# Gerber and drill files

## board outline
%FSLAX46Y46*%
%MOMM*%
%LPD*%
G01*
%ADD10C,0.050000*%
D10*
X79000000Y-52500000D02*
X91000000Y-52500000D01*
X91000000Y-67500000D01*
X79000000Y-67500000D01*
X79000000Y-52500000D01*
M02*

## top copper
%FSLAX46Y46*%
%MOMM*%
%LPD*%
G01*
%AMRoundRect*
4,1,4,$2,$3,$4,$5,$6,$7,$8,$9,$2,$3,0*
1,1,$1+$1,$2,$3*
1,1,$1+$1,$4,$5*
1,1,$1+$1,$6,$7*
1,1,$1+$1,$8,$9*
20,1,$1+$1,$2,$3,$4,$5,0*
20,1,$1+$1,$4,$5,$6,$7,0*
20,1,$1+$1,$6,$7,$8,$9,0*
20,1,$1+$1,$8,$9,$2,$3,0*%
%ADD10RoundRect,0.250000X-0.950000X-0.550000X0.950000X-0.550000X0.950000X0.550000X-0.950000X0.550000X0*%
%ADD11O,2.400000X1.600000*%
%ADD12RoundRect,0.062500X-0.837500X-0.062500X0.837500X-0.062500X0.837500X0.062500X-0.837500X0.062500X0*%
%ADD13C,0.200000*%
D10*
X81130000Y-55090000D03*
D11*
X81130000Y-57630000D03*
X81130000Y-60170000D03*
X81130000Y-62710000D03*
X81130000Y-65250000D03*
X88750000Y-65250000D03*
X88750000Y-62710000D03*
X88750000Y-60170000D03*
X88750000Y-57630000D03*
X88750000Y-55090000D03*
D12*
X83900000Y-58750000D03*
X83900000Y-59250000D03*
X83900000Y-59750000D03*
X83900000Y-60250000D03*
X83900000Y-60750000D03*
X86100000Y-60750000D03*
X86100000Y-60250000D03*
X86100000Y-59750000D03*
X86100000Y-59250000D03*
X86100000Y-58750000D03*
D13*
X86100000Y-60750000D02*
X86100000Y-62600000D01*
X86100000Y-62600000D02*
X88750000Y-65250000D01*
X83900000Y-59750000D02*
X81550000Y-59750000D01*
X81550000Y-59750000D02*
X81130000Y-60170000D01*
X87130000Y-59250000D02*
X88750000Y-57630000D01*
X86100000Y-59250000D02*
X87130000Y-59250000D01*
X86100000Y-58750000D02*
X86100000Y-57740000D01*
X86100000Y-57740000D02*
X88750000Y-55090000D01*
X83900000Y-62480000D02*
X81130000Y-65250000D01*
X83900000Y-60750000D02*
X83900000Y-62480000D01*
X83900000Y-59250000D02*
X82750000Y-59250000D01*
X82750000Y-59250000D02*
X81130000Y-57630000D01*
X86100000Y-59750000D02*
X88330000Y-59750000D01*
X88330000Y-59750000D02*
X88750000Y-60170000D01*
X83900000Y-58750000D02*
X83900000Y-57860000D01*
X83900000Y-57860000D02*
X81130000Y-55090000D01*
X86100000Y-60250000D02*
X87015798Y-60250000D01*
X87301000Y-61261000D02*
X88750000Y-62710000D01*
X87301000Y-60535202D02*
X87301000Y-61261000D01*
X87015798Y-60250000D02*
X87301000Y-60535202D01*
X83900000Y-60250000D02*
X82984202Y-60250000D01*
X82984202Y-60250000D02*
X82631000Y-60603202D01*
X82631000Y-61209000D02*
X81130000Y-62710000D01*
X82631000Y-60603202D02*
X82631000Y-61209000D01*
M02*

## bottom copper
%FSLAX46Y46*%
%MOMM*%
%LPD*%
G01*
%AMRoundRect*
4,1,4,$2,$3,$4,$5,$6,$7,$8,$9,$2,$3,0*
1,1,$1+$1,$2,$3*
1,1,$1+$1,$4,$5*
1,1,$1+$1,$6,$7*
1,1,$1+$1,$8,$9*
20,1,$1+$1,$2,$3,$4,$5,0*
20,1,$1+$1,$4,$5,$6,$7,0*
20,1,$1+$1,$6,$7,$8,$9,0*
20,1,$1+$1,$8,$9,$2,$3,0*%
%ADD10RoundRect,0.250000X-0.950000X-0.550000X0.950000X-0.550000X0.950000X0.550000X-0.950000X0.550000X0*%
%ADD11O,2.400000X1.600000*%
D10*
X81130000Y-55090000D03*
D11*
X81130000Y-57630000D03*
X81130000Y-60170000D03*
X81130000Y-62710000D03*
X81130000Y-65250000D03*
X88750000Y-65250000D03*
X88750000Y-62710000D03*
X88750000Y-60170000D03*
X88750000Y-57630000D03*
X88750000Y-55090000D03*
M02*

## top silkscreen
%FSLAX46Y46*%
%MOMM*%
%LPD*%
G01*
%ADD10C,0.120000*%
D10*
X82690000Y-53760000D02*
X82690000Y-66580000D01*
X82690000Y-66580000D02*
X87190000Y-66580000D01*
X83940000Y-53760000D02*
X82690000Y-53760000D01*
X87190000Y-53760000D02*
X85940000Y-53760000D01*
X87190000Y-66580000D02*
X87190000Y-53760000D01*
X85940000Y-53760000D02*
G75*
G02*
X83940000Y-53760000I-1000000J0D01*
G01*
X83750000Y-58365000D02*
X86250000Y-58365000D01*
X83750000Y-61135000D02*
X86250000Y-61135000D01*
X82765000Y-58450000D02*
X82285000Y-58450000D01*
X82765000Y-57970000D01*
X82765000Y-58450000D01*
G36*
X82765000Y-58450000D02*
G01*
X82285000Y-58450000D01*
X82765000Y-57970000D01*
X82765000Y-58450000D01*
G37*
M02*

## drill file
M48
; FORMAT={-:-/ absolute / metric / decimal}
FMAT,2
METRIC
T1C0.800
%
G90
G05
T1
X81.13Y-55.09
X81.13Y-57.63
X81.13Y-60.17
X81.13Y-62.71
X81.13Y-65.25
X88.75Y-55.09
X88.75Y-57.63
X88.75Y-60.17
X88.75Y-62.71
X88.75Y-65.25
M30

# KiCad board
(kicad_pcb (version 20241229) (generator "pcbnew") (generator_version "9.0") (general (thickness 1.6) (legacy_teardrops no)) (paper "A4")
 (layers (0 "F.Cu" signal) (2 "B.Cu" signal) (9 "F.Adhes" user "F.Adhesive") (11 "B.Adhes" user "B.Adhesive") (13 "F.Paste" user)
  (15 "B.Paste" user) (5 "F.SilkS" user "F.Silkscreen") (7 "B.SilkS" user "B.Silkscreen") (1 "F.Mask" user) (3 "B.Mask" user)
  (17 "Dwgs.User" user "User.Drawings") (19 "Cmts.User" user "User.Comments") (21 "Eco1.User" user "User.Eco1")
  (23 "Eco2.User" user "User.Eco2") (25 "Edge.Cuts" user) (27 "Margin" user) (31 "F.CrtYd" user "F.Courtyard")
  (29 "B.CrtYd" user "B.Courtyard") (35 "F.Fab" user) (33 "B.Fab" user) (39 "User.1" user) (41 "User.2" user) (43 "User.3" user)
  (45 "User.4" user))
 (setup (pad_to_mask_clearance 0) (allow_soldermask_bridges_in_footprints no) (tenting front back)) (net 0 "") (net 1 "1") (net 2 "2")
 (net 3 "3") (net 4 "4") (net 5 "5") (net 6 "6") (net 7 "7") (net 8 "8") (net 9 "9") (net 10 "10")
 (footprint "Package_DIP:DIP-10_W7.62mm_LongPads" (layer "F.Cu") (at 81.13 55.09)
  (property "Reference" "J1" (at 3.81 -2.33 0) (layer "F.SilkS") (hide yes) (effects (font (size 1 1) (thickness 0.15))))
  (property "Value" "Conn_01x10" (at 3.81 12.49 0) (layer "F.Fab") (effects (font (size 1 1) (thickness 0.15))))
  (fp_line (start 1.56 -1.33) (end 1.56 11.49) (stroke (width 0.12) (type solid)) (layer "F.SilkS"))
  (fp_line (start 1.56 11.49) (end 6.06 11.49) (stroke (width 0.12) (type solid)) (layer "F.SilkS"))
  (fp_line (start 2.81 -1.33) (end 1.56 -1.33) (stroke (width 0.12) (type solid)) (layer "F.SilkS"))
  (fp_line (start 6.06 -1.33) (end 4.81 -1.33) (stroke (width 0.12) (type solid)) (layer "F.SilkS"))
  (fp_line (start 6.06 11.49) (end 6.06 -1.33) (stroke (width 0.12) (type solid)) (layer "F.SilkS"))
  (fp_arc (start 4.81 -1.33) (mid 3.81 -0.33) (end 2.81 -1.33) (stroke (width 0.12) (type solid)) (layer "F.SilkS"))
  (pad "1" thru_hole roundrect (at 0 0) (size 2.4 1.6) (drill 0.8) (layers "*.Cu" "*.Mask") (remove_unused_layers no)
   (roundrect_rratio 0.15625) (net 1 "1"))
  (pad "2" thru_hole oval (at 0 2.54) (size 2.4 1.6) (drill 0.8) (layers "*.Cu" "*.Mask") (remove_unused_layers no) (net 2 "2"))
  (pad "3" thru_hole oval (at 0 5.08) (size 2.4 1.6) (drill 0.8) (layers "*.Cu" "*.Mask") (remove_unused_layers no) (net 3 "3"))
  (pad "4" thru_hole oval (at 0 7.62) (size 2.4 1.6) (drill 0.8) (layers "*.Cu" "*.Mask") (remove_unused_layers no) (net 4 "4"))
  (pad "5" thru_hole oval (at 0 10.16) (size 2.4 1.6) (drill 0.8) (layers "*.Cu" "*.Mask") (remove_unused_layers no) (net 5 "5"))
  (pad "6" thru_hole oval (at 7.62 10.16) (size 2.4 1.6) (drill 0.8) (layers "*.Cu" "*.Mask") (remove_unused_layers no) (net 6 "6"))
  (pad "7" thru_hole oval (at 7.62 7.62) (size 2.4 1.6) (drill 0.8) (layers "*.Cu" "*.Mask") (remove_unused_layers no) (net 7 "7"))
  (pad "8" thru_hole oval (at 7.62 5.08) (size 2.4 1.6) (drill 0.8) (layers "*.Cu" "*.Mask") (remove_unused_layers no) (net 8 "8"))
  (pad "9" thru_hole oval (at 7.62 2.54) (size 2.4 1.6) (drill 0.8) (layers "*.Cu" "*.Mask") (remove_unused_layers no) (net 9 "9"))
  (pad "10" thru_hole oval (at 7.62 0) (size 2.4 1.6) (drill 0.8) (layers "*.Cu" "*.Mask") (remove_unused_layers no) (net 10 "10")))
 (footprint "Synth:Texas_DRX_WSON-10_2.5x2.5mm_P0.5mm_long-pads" (layer "F.Cu") (at 85 59.75)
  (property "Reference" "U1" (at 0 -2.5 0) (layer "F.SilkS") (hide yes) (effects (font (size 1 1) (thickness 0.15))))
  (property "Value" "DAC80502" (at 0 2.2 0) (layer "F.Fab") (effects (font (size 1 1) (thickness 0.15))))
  (fp_line (start -1.25 -1.385) (end 1.25 -1.385) (stroke (width 0.12) (type solid)) (layer "F.SilkS"))
  (fp_line (start -1.25 1.385) (end 1.25 1.385) (stroke (width 0.12) (type solid)) (layer "F.SilkS"))
  (fp_poly
   (pts (xy -2.235 -1.3) (xy -2.715 -1.3) (xy -2.235 -1.78) (xy -2.235 -1.3)) (stroke (width 0.12) (type solid)) (fill yes)
   (layer "F.SilkS"))
  (pad "1" smd roundrect (at -1.1 -1) (size 1.8 0.25) (layers "F.Cu" "F.Mask" "F.Paste") (roundrect_rratio 0.25) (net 1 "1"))
  (pad "2" smd roundrect (at -1.1 -0.5) (size 1.8 0.25) (layers "F.Cu" "F.Mask" "F.Paste") (roundrect_rratio 0.25) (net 2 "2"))
  (pad "3" smd roundrect (at -1.1 0) (size 1.8 0.25) (layers "F.Cu" "F.Mask" "F.Paste") (roundrect_rratio 0.25) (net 3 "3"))
  (pad "4" smd roundrect (at -1.1 0.5) (size 1.8 0.25) (layers "F.Cu" "F.Mask" "F.Paste") (roundrect_rratio 0.25) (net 4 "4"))
  (pad "5" smd roundrect (at -1.1 1) (size 1.8 0.25) (layers "F.Cu" "F.Mask" "F.Paste") (roundrect_rratio 0.25) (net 5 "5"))
  (pad "6" smd roundrect (at 1.1 1) (size 1.8 0.25) (layers "F.Cu" "F.Mask" "F.Paste") (roundrect_rratio 0.25) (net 6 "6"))
  (pad "7" smd roundrect (at 1.1 0.5) (size 1.8 0.25) (layers "F.Cu" "F.Mask" "F.Paste") (roundrect_rratio 0.25) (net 7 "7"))
  (pad "8" smd roundrect (at 1.1 0) (size 1.8 0.25) (layers "F.Cu" "F.Mask" "F.Paste") (roundrect_rratio 0.25) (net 8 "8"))
  (pad "9" smd roundrect (at 1.1 -0.5) (size 1.8 0.25) (layers "F.Cu" "F.Mask" "F.Paste") (roundrect_rratio 0.25) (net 9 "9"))
  (pad "10" smd roundrect (at 1.1 -1) (size 1.8 0.25) (layers "F.Cu" "F.Mask" "F.Paste") (roundrect_rratio 0.25) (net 10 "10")))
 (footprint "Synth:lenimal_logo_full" (layer "B.Cu") (at 85 60 -90)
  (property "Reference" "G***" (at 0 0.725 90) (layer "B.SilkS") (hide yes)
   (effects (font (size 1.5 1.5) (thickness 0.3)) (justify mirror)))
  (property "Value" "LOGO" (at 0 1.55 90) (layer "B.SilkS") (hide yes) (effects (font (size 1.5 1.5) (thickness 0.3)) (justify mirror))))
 (gr_rect (start 79 52.5) (end 91 67.5) (stroke (width 0.05) (type default)) (fill no) (layer "Edge.Cuts"))
 (segment (start 86.1 60.75) (end 86.1 62.6) (width 0.2) (layer "F.Cu") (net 6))
 (segment (start 86.1 62.6) (end 88.75 65.25) (width 0.2) (layer "F.Cu") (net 6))
 (segment (start 83.9 59.75) (end 81.55 59.75) (width 0.2) (layer "F.Cu") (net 3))
 (segment (start 81.55 59.75) (end 81.13 60.17) (width 0.2) (layer "F.Cu") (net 3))
 (segment (start 87.13 59.25) (end 88.75 57.63) (width 0.2) (layer "F.Cu") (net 9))
 (segment (start 86.1 59.25) (end 87.13 59.25) (width 0.2) (layer "F.Cu") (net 9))
 (segment (start 86.1 58.75) (end 86.1 57.74) (width 0.2) (layer "F.Cu") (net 10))
 (segment (start 86.1 57.74) (end 88.75 55.09) (width 0.2) (layer "F.Cu") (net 10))
 (segment (start 83.9 62.48) (end 81.13 65.25) (width 0.2) (layer "F.Cu") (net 5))
 (segment (start 83.9 60.75) (end 83.9 62.48) (width 0.2) (layer "F.Cu") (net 5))
 (segment (start 83.9 59.25) (end 82.75 59.25) (width 0.2) (layer "F.Cu") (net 2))
 (segment (start 82.75 59.25) (end 81.13 57.63) (width 0.2) (layer "F.Cu") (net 2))
 (segment (start 86.1 59.75) (end 88.33 59.75) (width 0.2) (layer "F.Cu") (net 8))
 (segment (start 88.33 59.75) (end 88.75 60.17) (width 0.2) (layer "F.Cu") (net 8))
 (segment (start 83.9 58.75) (end 83.9 57.86) (width 0.2) (layer "F.Cu") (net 1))
 (segment (start 83.9 57.86) (end 81.13 55.09) (width 0.2) (layer "F.Cu") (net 1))
 (segment (start 86.1 60.25) (end 87.015798 60.25) (width 0.2) (layer "F.Cu") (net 7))
 (segment (start 87.301 61.261) (end 88.75 62.71) (width 0.2) (layer "F.Cu") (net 7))
 (segment (start 87.301 60.535202) (end 87.301 61.261) (width 0.2) (layer "F.Cu") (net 7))
 (segment (start 87.015798 60.25) (end 87.301 60.535202) (width 0.2) (layer "F.Cu") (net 7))
 (segment (start 83.9 60.25) (end 82.984202 60.25) (width 0.2) (layer "F.Cu") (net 4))
 (segment (start 82.984202 60.25) (end 82.631 60.603202) (width 0.2) (layer "F.Cu") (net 4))
 (segment (start 82.631 61.209) (end 81.13 62.71) (width 0.2) (layer "F.Cu") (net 4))
 (segment (start 82.631 60.603202) (end 82.631 61.209) (width 0.2) (layer "F.Cu") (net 4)))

